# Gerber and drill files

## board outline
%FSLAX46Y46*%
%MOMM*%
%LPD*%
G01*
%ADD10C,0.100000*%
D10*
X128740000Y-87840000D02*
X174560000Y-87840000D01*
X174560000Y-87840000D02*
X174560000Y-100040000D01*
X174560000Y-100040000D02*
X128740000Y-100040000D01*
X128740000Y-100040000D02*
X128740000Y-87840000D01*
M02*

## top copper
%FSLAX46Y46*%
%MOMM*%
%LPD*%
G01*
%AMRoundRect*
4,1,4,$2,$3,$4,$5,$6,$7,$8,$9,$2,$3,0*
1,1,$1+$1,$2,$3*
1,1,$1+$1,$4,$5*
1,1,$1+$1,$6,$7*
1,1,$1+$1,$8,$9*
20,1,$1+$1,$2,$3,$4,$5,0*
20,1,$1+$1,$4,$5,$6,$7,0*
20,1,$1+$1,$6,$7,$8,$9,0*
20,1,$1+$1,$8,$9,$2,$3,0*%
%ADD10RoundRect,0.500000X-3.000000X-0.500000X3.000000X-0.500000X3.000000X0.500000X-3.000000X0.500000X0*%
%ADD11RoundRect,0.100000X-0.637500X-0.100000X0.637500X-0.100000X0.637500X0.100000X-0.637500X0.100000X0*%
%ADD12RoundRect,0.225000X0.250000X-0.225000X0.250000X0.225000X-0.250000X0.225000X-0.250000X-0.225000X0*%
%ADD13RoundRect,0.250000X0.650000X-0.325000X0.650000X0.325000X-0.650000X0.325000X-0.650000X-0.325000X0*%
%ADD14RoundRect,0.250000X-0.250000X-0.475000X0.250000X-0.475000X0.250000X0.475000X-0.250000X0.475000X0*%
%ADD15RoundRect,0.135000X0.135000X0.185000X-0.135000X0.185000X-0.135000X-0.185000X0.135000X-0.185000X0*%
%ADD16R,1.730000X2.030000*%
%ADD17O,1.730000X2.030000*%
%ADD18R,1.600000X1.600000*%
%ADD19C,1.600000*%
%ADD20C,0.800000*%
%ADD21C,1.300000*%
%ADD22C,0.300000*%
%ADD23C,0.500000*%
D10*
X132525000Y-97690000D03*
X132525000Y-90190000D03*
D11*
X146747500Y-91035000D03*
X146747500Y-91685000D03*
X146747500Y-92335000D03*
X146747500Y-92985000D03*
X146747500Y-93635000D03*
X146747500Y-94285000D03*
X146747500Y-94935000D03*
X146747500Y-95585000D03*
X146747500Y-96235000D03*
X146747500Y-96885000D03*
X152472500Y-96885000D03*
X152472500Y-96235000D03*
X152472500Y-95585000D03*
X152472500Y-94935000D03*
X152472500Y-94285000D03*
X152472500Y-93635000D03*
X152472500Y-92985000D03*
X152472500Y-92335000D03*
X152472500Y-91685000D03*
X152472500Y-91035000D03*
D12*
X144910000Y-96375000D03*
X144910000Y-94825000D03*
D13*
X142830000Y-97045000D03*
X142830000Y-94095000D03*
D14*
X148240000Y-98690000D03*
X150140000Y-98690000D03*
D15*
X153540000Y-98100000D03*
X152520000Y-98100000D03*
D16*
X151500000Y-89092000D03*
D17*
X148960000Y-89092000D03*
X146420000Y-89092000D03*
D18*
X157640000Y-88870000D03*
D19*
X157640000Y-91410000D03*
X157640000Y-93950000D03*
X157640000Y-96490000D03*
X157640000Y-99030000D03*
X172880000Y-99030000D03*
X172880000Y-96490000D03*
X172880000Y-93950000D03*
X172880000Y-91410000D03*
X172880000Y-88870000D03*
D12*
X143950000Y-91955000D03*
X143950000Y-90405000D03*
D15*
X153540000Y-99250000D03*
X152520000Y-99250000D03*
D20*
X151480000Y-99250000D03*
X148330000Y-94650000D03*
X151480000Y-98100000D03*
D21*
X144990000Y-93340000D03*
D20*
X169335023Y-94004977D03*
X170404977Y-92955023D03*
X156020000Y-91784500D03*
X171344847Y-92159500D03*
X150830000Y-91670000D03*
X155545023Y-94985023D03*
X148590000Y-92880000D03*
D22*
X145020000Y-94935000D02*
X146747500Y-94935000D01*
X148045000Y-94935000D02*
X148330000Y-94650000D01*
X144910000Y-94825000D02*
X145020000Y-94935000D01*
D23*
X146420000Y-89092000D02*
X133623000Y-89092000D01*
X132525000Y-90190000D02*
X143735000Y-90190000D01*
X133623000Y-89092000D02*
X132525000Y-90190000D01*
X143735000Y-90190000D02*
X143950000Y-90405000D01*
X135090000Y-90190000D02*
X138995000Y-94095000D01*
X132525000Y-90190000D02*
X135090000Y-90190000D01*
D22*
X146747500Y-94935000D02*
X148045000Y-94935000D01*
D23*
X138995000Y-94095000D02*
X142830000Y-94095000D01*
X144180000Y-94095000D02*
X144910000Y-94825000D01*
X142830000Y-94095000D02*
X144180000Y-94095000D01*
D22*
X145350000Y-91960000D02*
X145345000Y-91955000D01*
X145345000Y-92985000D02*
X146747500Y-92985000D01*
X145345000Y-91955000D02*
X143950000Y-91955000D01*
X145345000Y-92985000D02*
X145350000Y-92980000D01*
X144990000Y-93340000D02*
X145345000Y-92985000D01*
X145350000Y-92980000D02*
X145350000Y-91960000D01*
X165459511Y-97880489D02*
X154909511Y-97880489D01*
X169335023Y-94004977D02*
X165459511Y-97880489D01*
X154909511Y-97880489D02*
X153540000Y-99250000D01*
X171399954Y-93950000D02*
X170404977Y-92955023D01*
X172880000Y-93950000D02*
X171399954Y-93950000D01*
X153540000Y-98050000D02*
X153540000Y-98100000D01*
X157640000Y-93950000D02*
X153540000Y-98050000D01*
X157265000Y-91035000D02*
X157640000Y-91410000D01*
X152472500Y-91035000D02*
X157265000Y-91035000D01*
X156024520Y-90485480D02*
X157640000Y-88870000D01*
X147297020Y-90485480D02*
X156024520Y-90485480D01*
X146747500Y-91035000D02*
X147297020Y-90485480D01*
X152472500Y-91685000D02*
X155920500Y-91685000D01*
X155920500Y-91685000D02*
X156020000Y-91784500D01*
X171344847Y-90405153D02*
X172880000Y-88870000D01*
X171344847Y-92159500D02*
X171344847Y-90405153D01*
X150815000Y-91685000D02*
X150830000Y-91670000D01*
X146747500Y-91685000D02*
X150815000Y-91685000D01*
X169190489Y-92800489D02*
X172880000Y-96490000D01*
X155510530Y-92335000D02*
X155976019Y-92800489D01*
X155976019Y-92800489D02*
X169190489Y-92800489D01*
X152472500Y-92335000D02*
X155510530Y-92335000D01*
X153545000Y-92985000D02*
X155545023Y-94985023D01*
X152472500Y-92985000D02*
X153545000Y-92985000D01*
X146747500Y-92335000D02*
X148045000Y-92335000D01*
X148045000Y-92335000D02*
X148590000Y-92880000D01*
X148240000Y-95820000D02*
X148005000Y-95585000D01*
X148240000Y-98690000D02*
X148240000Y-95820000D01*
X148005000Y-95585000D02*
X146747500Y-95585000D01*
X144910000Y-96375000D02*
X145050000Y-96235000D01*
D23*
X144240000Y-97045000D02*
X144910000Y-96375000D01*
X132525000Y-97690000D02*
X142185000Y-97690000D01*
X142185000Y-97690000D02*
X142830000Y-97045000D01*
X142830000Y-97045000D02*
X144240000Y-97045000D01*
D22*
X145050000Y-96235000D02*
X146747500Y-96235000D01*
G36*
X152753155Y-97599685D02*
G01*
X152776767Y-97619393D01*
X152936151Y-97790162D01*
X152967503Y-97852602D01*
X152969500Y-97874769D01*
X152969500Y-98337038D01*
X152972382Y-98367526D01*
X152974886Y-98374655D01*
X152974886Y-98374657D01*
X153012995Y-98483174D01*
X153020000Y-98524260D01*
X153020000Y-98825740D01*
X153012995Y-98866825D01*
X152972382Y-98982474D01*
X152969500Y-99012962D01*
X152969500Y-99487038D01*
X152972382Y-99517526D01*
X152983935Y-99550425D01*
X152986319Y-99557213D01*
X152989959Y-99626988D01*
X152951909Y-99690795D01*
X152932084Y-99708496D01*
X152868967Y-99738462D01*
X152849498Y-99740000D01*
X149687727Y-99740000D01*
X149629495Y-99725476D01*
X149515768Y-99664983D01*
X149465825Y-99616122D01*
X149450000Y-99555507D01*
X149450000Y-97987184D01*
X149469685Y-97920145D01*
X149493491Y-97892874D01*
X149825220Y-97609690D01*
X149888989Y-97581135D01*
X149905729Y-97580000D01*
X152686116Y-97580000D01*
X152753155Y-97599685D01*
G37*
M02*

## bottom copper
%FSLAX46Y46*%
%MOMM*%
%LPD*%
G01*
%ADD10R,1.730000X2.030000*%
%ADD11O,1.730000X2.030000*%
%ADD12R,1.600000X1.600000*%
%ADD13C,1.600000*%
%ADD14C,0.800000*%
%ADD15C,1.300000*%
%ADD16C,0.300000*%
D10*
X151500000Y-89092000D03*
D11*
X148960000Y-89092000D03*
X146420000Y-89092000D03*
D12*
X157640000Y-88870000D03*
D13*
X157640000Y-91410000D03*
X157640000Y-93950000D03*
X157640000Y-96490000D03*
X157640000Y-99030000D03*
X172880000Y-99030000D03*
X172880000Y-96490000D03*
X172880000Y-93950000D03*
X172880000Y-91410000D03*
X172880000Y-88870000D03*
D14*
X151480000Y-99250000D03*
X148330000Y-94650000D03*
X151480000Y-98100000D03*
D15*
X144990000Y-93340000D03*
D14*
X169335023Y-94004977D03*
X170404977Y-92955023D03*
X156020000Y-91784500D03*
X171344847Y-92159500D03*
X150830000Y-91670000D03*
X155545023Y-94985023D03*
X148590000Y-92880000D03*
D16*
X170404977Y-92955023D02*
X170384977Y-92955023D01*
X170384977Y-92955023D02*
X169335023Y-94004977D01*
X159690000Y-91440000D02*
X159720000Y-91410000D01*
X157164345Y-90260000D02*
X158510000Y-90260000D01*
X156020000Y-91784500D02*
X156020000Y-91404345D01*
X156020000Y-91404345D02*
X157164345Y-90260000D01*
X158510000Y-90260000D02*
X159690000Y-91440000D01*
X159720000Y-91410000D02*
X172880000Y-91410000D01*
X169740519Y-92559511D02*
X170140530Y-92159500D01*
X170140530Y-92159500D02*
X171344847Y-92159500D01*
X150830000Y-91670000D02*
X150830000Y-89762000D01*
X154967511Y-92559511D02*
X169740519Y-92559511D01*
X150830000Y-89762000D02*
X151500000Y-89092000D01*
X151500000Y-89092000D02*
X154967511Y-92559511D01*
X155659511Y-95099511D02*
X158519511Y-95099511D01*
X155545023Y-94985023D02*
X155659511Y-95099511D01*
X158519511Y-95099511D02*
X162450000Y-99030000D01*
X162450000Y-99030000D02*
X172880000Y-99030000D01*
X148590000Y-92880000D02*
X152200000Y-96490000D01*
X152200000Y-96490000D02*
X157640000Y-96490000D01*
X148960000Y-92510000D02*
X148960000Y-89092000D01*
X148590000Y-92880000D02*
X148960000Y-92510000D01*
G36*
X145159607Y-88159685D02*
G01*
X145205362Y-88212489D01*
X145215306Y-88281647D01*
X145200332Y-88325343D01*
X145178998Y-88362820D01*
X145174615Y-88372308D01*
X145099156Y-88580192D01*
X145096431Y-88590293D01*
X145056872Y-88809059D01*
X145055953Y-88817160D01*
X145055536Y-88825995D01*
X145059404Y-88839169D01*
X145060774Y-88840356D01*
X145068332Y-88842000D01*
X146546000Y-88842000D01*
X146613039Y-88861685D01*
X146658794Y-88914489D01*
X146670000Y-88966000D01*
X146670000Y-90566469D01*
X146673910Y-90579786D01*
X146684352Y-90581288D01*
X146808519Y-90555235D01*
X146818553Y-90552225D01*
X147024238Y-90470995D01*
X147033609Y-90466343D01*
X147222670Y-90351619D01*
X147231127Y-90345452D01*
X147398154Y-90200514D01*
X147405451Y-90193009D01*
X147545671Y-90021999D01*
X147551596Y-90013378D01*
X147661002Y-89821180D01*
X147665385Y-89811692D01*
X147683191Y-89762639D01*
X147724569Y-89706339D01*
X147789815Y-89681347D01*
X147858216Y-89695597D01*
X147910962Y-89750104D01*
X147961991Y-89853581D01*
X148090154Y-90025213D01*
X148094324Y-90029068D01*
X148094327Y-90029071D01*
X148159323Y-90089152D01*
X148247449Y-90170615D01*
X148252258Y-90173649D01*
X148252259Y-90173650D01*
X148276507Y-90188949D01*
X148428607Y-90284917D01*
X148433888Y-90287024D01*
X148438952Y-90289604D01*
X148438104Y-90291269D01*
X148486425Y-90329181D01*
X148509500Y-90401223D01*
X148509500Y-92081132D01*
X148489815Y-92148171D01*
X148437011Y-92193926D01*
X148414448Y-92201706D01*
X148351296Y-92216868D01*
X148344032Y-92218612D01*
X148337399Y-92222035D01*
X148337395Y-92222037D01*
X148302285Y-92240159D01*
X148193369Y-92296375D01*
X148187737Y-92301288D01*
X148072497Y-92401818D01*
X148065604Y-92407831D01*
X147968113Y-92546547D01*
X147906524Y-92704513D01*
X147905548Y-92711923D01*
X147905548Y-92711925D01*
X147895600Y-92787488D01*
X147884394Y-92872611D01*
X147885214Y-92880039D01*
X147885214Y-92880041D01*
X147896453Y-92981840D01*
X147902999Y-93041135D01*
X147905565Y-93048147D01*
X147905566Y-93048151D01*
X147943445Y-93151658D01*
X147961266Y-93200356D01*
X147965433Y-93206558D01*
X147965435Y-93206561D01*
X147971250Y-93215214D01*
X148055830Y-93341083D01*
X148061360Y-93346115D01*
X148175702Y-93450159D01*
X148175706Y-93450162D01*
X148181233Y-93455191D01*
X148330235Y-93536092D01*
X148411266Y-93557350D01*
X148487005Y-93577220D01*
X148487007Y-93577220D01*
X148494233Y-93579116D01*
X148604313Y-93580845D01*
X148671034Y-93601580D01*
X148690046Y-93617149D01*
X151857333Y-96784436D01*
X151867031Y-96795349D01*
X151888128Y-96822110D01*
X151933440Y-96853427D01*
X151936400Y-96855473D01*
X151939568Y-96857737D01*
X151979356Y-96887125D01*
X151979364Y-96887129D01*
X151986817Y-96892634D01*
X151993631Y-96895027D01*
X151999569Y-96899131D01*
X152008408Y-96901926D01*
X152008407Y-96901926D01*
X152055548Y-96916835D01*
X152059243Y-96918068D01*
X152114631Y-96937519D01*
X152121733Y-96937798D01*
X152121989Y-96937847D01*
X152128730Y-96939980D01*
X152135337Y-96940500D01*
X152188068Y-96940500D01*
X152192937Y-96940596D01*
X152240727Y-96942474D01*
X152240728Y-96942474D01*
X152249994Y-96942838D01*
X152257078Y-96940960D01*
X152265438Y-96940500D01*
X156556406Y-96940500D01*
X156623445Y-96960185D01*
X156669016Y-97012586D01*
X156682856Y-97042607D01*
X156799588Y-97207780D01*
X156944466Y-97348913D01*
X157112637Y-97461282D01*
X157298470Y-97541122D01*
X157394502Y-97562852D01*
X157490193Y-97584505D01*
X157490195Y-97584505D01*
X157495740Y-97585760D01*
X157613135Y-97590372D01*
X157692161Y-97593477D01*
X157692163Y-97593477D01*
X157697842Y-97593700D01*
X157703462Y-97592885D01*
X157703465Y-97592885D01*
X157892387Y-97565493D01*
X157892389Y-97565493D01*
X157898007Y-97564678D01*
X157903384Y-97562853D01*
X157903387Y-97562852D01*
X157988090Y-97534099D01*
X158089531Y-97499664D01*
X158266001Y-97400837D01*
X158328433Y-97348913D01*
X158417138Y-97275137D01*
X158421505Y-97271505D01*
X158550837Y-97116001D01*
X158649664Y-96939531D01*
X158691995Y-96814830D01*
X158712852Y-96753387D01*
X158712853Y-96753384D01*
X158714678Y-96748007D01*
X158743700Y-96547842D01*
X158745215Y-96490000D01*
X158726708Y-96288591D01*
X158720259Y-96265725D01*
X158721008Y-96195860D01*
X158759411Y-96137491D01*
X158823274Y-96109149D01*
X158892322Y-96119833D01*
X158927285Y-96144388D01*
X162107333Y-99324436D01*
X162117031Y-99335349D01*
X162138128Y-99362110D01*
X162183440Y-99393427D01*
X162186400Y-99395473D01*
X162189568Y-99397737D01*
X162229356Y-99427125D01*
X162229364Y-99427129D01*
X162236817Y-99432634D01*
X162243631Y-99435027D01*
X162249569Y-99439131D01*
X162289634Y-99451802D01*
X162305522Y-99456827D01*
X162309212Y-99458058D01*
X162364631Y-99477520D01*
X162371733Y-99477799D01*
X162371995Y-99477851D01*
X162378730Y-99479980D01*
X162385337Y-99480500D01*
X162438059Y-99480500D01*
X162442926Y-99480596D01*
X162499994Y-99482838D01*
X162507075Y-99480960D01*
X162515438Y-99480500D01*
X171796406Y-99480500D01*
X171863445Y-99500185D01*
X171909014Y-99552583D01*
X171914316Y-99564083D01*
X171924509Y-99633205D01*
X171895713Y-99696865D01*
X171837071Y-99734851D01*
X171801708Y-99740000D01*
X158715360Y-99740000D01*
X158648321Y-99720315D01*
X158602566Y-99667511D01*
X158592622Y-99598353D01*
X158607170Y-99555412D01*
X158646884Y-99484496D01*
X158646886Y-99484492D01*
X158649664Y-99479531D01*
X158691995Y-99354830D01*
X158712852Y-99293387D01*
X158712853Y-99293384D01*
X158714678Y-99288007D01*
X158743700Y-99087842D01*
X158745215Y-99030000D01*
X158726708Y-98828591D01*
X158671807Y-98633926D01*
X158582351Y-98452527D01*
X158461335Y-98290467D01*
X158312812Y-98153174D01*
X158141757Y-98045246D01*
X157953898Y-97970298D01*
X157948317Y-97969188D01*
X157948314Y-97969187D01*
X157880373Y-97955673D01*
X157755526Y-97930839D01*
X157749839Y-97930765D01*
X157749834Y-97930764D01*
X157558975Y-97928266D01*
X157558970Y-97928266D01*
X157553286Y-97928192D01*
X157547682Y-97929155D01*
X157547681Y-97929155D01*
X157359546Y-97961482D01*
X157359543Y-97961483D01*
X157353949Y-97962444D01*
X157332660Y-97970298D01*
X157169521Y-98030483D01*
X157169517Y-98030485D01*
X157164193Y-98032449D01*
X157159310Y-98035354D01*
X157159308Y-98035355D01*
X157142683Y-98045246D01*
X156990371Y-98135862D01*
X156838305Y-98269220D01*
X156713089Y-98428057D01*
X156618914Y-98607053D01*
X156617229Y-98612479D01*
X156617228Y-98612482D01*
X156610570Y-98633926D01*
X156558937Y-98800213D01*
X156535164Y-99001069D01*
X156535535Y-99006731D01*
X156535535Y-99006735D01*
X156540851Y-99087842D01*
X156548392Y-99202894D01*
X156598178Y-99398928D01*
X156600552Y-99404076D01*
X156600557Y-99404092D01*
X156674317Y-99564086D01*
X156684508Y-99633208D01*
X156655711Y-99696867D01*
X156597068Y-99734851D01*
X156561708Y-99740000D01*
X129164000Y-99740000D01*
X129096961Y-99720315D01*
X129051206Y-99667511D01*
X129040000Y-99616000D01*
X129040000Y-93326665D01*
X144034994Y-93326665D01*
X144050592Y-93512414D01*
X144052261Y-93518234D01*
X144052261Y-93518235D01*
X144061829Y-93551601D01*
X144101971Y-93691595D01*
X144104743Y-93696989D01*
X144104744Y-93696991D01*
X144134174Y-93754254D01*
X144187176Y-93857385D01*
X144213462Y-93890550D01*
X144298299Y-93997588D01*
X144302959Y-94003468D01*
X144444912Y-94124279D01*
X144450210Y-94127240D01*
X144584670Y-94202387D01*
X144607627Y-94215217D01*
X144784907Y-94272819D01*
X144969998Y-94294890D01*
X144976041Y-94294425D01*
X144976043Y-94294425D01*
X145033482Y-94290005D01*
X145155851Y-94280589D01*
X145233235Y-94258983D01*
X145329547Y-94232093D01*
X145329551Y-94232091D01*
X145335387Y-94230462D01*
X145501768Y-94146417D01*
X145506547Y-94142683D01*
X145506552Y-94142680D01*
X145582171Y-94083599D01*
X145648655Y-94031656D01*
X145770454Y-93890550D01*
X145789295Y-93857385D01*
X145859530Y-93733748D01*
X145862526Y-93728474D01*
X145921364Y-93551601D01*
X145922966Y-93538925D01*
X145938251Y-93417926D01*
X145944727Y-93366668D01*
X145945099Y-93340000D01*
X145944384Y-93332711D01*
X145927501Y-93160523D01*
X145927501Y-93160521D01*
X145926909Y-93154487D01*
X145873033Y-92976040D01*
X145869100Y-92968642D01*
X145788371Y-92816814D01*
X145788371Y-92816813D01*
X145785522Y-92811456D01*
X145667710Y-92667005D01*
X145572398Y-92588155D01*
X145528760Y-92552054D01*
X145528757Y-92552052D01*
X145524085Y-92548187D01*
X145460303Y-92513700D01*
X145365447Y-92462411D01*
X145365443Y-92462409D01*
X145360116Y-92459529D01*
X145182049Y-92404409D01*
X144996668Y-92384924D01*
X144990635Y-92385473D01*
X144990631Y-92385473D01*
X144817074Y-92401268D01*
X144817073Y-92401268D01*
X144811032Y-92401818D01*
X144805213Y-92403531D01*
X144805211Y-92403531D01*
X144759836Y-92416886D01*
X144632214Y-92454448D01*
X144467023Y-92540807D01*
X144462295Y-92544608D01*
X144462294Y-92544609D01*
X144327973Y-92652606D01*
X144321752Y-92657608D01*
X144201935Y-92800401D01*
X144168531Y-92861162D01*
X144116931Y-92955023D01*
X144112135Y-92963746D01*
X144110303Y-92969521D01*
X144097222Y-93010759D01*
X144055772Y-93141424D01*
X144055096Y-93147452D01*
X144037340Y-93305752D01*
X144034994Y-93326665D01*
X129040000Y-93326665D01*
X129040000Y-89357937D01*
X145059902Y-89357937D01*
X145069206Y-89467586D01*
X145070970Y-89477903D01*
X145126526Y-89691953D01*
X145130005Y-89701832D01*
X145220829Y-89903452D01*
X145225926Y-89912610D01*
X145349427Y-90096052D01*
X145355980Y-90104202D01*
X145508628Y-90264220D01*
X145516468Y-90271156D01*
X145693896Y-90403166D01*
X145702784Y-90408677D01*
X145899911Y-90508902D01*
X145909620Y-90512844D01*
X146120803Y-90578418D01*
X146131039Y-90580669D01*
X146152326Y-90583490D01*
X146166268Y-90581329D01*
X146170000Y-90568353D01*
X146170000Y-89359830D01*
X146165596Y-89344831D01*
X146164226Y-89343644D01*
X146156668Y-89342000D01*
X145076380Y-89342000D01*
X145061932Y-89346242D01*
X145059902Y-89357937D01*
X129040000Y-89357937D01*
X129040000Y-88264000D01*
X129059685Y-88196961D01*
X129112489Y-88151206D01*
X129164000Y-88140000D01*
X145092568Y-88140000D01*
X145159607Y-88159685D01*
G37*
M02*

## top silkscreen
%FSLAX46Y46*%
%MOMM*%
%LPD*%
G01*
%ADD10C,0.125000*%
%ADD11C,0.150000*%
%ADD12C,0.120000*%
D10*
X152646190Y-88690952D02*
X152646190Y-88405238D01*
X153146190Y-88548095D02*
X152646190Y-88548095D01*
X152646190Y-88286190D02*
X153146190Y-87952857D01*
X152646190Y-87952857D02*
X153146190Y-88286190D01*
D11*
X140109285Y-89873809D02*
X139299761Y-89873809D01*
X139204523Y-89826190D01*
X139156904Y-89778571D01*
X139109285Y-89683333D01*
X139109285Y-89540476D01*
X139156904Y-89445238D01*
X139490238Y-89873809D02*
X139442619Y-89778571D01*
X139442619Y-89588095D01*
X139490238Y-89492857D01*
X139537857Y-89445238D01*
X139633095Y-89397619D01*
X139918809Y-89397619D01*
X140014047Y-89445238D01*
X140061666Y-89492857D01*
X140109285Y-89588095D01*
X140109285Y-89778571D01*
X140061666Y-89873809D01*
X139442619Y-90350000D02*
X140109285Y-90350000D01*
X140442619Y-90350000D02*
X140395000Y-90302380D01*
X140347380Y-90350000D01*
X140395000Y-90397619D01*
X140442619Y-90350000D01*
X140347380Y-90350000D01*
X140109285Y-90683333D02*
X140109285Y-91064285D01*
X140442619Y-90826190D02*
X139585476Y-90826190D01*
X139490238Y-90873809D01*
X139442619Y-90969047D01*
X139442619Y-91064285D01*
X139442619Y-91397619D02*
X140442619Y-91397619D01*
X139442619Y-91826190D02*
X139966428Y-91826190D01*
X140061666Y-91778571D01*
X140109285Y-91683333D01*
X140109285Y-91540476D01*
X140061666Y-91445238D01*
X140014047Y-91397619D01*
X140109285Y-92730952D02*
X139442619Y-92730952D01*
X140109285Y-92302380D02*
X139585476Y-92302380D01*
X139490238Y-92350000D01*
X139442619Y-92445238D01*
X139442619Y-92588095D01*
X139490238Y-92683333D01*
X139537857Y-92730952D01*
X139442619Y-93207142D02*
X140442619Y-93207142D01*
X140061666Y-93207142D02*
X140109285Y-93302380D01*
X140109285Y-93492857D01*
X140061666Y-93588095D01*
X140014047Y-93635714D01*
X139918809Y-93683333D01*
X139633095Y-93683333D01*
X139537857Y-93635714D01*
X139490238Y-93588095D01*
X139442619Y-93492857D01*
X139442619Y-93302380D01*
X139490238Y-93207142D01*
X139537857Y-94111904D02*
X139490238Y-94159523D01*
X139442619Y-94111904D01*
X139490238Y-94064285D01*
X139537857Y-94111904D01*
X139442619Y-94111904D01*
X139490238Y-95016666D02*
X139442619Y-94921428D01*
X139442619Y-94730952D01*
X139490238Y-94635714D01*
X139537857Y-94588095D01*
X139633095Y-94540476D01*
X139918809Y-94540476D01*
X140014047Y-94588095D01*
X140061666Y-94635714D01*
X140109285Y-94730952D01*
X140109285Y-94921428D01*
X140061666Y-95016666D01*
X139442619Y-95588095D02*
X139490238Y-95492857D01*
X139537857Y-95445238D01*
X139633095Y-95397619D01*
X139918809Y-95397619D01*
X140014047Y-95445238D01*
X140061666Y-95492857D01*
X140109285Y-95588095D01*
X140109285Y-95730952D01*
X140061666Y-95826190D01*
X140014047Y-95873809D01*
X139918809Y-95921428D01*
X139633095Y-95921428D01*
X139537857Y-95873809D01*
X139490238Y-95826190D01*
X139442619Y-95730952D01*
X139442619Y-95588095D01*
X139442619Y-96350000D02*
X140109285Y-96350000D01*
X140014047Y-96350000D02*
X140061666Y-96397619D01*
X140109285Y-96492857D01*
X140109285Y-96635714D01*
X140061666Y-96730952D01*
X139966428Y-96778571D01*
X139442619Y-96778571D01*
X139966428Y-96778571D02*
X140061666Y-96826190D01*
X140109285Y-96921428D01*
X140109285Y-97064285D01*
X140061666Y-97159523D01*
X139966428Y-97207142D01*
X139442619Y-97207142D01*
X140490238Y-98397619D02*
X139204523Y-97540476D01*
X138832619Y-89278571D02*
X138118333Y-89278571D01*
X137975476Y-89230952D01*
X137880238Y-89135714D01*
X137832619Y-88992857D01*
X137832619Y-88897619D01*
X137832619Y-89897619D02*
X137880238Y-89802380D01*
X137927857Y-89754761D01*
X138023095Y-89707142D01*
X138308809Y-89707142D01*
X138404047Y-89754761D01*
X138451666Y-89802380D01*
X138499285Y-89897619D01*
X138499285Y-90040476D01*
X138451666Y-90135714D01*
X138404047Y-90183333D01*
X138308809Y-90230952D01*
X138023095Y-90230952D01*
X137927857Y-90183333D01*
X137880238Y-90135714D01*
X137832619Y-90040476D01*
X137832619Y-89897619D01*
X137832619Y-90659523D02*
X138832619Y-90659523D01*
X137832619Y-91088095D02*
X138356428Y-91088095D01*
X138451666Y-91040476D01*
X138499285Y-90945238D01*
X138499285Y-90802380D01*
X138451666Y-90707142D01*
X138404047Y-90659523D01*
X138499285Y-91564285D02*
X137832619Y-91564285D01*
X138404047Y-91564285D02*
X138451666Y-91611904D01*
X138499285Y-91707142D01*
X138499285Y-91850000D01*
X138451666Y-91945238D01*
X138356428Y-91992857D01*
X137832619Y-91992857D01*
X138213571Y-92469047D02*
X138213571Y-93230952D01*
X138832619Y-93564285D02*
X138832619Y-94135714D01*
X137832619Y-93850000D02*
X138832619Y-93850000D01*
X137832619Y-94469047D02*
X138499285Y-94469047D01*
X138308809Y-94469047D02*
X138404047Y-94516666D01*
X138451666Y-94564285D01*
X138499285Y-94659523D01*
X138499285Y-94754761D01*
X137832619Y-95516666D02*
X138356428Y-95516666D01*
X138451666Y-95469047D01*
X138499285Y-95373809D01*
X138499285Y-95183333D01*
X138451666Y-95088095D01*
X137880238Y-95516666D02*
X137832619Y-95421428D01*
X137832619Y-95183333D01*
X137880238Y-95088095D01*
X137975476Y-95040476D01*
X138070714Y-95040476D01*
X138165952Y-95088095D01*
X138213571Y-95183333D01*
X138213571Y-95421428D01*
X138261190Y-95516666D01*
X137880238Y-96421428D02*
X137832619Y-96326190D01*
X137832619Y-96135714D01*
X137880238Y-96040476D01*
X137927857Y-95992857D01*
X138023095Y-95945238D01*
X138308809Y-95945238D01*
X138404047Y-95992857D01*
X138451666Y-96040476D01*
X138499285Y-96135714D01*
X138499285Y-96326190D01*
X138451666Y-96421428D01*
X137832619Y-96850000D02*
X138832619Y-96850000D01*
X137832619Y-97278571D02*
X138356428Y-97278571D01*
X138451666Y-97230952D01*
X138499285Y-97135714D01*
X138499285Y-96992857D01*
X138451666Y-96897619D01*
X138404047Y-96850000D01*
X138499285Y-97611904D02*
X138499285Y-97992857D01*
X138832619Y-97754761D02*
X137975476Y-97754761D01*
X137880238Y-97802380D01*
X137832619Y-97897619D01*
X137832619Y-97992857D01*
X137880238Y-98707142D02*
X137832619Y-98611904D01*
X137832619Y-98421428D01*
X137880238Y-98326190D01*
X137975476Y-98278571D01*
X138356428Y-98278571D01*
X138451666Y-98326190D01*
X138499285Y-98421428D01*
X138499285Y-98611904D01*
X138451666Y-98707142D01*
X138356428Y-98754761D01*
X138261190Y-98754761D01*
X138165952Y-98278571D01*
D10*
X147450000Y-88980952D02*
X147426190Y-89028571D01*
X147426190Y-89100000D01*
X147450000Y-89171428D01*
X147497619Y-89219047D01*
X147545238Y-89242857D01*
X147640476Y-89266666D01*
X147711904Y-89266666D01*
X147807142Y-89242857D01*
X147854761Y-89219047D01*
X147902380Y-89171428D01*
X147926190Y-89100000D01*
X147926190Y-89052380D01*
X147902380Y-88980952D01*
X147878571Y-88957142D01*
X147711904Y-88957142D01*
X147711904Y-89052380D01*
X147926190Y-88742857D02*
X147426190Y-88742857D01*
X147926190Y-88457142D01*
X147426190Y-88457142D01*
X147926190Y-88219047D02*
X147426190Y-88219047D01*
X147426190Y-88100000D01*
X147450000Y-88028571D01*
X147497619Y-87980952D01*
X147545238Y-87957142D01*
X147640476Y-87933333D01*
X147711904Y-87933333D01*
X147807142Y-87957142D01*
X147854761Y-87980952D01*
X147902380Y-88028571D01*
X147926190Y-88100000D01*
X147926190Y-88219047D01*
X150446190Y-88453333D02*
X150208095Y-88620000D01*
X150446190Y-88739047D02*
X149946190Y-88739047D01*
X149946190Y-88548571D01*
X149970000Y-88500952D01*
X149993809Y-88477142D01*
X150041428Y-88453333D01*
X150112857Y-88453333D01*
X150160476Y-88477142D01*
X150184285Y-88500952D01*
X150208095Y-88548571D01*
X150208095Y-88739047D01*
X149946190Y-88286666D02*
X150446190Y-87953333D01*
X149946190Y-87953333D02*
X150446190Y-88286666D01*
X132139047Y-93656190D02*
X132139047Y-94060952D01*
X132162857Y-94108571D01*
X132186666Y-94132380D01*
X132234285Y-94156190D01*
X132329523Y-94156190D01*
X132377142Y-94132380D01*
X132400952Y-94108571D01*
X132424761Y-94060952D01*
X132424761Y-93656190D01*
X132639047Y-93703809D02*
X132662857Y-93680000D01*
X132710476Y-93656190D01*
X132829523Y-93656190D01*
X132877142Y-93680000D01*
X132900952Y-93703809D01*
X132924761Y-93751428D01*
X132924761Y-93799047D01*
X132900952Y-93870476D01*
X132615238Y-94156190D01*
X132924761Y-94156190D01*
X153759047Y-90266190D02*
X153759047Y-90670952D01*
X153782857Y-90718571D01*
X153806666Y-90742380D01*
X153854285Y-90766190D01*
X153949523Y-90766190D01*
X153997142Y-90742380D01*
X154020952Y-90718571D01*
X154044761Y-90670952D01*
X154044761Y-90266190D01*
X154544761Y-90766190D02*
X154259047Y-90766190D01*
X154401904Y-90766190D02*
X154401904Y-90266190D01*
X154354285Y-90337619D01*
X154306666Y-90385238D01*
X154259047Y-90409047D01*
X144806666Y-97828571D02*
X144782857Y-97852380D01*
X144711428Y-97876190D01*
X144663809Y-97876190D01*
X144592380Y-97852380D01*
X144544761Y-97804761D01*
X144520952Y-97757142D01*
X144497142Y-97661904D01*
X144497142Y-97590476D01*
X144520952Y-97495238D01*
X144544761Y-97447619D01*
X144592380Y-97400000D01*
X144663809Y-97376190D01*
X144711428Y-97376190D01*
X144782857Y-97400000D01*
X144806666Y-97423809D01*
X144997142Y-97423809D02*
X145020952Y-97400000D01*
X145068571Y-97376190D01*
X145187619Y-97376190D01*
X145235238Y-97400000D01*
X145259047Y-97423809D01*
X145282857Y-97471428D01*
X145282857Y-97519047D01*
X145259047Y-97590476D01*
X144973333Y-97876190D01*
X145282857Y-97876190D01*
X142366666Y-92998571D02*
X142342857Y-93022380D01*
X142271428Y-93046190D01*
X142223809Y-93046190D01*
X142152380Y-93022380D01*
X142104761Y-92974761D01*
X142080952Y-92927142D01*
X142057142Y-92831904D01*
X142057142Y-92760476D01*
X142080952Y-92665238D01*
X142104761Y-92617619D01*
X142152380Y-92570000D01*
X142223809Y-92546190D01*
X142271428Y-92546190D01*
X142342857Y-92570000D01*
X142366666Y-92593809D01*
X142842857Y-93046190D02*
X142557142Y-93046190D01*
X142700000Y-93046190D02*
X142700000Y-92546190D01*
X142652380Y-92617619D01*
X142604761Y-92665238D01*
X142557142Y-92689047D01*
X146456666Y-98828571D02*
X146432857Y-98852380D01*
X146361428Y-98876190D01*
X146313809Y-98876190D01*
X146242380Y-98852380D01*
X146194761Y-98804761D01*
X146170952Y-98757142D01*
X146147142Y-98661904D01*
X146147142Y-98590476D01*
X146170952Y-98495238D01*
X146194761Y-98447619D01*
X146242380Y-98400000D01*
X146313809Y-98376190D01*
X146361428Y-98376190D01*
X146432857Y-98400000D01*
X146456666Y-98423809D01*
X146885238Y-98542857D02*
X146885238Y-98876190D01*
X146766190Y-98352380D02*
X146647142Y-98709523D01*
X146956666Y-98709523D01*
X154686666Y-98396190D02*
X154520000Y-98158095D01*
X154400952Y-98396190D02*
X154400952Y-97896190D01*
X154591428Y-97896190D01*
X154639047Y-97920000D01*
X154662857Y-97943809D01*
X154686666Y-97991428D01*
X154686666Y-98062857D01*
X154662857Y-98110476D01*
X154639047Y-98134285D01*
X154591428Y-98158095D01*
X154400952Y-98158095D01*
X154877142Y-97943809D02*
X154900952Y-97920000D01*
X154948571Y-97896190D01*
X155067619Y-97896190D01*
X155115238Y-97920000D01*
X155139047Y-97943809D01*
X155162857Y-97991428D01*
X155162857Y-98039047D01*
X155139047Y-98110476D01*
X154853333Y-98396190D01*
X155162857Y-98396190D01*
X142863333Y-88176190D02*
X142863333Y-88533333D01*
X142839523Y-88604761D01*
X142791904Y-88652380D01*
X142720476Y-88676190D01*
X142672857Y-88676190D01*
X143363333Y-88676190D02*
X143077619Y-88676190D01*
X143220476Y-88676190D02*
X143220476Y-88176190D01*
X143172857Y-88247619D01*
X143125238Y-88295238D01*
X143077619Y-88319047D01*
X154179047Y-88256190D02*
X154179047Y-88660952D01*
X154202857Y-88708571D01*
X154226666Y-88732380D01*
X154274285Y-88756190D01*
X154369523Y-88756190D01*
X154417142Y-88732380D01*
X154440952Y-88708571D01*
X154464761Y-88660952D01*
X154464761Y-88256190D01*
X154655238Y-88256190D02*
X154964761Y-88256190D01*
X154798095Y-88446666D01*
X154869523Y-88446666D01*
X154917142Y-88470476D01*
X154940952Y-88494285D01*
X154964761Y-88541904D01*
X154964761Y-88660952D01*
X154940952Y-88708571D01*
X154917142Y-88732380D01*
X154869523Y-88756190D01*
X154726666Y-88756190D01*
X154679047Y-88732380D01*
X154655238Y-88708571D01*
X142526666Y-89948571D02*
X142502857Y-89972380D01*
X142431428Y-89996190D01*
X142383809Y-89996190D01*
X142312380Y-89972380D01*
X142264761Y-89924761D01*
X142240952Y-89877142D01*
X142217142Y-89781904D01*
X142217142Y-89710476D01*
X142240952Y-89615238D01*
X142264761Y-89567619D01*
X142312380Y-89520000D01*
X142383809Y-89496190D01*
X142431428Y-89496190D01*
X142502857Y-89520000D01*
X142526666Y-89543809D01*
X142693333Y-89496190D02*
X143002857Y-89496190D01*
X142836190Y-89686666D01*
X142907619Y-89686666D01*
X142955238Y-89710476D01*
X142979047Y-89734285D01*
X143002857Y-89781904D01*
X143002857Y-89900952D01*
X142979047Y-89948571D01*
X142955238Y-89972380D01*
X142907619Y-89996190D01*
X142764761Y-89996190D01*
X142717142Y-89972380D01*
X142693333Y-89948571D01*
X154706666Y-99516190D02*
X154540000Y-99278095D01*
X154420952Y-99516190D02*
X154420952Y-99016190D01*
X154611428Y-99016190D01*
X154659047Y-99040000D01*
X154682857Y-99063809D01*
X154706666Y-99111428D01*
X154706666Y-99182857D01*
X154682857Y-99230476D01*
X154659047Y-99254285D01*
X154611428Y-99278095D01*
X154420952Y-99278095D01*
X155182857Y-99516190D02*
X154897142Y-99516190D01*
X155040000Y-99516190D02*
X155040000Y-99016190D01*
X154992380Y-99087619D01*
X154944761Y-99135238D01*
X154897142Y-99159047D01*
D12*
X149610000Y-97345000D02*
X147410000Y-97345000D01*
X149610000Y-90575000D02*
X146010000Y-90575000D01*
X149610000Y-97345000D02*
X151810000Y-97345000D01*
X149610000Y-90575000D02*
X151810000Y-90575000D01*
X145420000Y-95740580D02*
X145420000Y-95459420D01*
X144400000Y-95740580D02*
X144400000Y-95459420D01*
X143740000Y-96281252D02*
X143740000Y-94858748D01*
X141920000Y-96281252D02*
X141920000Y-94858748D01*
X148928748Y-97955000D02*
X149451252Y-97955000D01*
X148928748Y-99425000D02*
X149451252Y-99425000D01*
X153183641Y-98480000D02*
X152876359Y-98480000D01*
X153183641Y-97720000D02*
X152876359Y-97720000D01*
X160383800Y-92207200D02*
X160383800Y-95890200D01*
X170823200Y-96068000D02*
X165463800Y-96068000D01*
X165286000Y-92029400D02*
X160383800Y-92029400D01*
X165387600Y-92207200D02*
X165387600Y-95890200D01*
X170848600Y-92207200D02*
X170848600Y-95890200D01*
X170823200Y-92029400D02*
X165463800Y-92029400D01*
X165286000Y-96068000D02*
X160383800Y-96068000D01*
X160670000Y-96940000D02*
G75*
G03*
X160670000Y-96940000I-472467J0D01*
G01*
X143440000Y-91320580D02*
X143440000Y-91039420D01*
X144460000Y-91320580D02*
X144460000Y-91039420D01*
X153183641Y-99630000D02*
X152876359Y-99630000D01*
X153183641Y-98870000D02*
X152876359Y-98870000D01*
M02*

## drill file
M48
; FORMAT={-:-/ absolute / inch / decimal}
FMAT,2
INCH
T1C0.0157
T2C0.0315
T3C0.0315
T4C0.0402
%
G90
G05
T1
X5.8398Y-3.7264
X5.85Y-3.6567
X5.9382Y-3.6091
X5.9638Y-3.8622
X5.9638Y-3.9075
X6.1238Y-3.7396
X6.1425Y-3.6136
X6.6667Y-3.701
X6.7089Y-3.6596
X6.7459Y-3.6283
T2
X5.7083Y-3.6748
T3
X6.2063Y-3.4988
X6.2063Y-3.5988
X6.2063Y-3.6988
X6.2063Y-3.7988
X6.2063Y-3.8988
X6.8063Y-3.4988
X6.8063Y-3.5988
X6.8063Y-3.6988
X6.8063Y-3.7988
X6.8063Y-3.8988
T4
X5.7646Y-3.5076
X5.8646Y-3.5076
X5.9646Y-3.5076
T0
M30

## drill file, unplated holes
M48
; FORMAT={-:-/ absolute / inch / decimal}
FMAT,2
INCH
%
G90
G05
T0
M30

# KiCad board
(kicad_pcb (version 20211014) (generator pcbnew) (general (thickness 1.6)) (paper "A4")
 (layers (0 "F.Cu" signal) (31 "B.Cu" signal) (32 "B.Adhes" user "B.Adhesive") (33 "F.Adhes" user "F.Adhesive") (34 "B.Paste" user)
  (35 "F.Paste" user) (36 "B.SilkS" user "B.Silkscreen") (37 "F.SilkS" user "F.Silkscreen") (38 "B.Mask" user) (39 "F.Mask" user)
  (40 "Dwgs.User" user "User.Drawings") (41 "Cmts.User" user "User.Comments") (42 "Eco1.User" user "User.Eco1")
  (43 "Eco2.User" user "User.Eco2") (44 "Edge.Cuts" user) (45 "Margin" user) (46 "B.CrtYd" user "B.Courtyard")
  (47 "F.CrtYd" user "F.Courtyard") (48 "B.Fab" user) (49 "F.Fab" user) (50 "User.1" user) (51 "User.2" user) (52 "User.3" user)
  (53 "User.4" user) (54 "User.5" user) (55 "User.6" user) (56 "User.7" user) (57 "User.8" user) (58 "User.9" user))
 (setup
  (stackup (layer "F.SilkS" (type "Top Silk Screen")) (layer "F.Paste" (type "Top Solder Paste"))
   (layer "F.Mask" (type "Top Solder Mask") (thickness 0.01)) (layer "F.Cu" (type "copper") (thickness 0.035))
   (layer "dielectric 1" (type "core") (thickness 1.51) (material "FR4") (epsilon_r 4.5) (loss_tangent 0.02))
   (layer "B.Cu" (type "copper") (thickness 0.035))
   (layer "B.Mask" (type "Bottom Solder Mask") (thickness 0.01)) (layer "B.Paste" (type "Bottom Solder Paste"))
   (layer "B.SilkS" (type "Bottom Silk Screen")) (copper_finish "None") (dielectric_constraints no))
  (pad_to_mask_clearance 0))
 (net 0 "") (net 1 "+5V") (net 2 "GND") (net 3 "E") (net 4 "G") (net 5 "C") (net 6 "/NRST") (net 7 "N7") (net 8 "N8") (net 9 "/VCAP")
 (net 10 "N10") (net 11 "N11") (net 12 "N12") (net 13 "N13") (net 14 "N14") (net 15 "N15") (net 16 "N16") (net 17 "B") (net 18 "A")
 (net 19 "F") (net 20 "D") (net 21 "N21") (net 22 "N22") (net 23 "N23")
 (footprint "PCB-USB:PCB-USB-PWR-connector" (layer "F.Cu") (at 132.525 93.94)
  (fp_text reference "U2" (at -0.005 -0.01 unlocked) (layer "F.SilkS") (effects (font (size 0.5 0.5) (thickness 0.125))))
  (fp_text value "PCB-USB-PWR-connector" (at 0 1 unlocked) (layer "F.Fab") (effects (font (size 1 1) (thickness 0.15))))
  (pad "1" smd roundrect (at 0 3.75) (size 7 2) (layers "F.Cu" "F.Paste" "F.Mask") (roundrect_rratio 0.25) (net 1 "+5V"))
  (pad "2" smd roundrect (at 0 -3.75) (size 7 2) (layers "F.Cu" "F.Paste" "F.Mask") (roundrect_rratio 0.25) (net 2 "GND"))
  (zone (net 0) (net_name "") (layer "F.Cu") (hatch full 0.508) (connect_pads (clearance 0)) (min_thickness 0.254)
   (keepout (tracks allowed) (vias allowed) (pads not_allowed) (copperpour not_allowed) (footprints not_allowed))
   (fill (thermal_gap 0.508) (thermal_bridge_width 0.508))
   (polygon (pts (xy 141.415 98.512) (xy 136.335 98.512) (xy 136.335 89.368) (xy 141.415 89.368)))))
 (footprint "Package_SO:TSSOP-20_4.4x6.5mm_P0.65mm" (layer "F.Cu") (at 149.61 93.96)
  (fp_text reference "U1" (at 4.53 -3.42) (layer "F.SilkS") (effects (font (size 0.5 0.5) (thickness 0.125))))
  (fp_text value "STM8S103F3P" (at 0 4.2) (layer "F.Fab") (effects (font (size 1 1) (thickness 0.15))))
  (fp_line (start 0 3.385) (end -2.2 3.385) (layer "F.SilkS") (width 0.12))
  (fp_line (start 0 -3.385) (end -3.6 -3.385) (layer "F.SilkS") (width 0.12))
  (fp_line (start 0 3.385) (end 2.2 3.385) (layer "F.SilkS") (width 0.12))
  (fp_line (start 0 -3.385) (end 2.2 -3.385) (layer "F.SilkS") (width 0.12))
  (pad "1" smd roundrect (at -2.8625 -2.925) (size 1.475 0.4) (layers "F.Cu" "F.Paste" "F.Mask") (roundrect_rratio 0.25) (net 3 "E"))
  (pad "2" smd roundrect (at -2.8625 -2.275) (size 1.475 0.4) (layers "F.Cu" "F.Paste" "F.Mask") (roundrect_rratio 0.25) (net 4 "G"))
  (pad "3" smd roundrect (at -2.8625 -1.625) (size 1.475 0.4) (layers "F.Cu" "F.Paste" "F.Mask") (roundrect_rratio 0.25) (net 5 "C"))
  (pad "4" smd roundrect (at -2.8625 -0.975) (size 1.475 0.4) (layers "F.Cu" "F.Paste" "F.Mask") (roundrect_rratio 0.25) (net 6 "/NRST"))
  (pad "5" smd roundrect (at -2.8625 -0.325) (size 1.475 0.4) (layers "F.Cu" "F.Paste" "F.Mask") (roundrect_rratio 0.25) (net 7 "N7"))
  (pad "6" smd roundrect (at -2.8625 0.325) (size 1.475 0.4) (layers "F.Cu" "F.Paste" "F.Mask") (roundrect_rratio 0.25) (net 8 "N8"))
  (pad "7" smd roundrect (at -2.8625 0.975) (size 1.475 0.4) (layers "F.Cu" "F.Paste" "F.Mask") (roundrect_rratio 0.25) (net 2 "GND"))
  (pad "8" smd roundrect (at -2.8625 1.625) (size 1.475 0.4) (layers "F.Cu" "F.Paste" "F.Mask") (roundrect_rratio 0.25) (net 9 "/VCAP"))
  (pad "9" smd roundrect (at -2.8625 2.275) (size 1.475 0.4) (layers "F.Cu" "F.Paste" "F.Mask") (roundrect_rratio 0.25) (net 1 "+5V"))
  (pad "10" smd roundrect (at -2.8625 2.925) (size 1.475 0.4) (layers "F.Cu" "F.Paste" "F.Mask") (roundrect_rratio 0.25) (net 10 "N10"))
  (pad "11" smd roundrect (at 2.8625 2.925) (size 1.475 0.4) (layers "F.Cu" "F.Paste" "F.Mask") (roundrect_rratio 0.25) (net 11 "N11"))
  (pad "12" smd roundrect (at 2.8625 2.275) (size 1.475 0.4) (layers "F.Cu" "F.Paste" "F.Mask") (roundrect_rratio 0.25) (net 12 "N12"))
  (pad "13" smd roundrect (at 2.8625 1.625) (size 1.475 0.4) (layers "F.Cu" "F.Paste" "F.Mask") (roundrect_rratio 0.25) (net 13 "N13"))
  (pad "14" smd roundrect (at 2.8625 0.975) (size 1.475 0.4) (layers "F.Cu" "F.Paste" "F.Mask") (roundrect_rratio 0.25) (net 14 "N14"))
  (pad "15" smd roundrect (at 2.8625 0.325) (size 1.475 0.4) (layers "F.Cu" "F.Paste" "F.Mask") (roundrect_rratio 0.25) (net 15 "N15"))
  (pad "16" smd roundrect (at 2.8625 -0.325) (size 1.475 0.4) (layers "F.Cu" "F.Paste" "F.Mask") (roundrect_rratio 0.25) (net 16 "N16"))
  (pad "17" smd roundrect (at 2.8625 -0.975) (size 1.475 0.4) (layers "F.Cu" "F.Paste" "F.Mask") (roundrect_rratio 0.25) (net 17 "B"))
  (pad "18" smd roundrect (at 2.8625 -1.625) (size 1.475 0.4) (layers "F.Cu" "F.Paste" "F.Mask") (roundrect_rratio 0.25) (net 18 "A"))
  (pad "19" smd roundrect (at 2.8625 -2.275) (size 1.475 0.4) (layers "F.Cu" "F.Paste" "F.Mask") (roundrect_rratio 0.25) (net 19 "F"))
  (pad "20" smd roundrect (at 2.8625 -2.925) (size 1.475 0.4) (layers "F.Cu" "F.Paste" "F.Mask") (roundrect_rratio 0.25) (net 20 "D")))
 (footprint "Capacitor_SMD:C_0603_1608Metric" (layer "F.Cu") (at 144.91 95.6 90)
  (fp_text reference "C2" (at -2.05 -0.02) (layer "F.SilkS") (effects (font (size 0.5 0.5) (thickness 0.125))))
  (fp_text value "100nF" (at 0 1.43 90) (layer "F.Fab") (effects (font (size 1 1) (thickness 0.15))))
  (fp_line (start -0.14058 0.51) (end 0.14058 0.51) (layer "F.SilkS") (width 0.12))
  (fp_line (start -0.14058 -0.51) (end 0.14058 -0.51) (layer "F.SilkS") (width 0.12))
  (pad "1" smd roundrect (at -0.775 0 90) (size 0.9 0.95) (layers "F.Cu" "F.Paste" "F.Mask") (roundrect_rratio 0.25) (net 1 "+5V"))
  (pad "2" smd roundrect (at 0.775 0 90) (size 0.9 0.95) (layers "F.Cu" "F.Paste" "F.Mask") (roundrect_rratio 0.25) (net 2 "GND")))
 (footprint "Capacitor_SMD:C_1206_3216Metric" (layer "F.Cu") (at 142.83 95.57 90)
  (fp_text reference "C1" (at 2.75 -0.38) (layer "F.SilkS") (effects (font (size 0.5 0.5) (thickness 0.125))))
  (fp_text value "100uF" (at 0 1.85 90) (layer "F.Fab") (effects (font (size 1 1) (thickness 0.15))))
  (fp_line (start -0.711252 0.91) (end 0.711252 0.91) (layer "F.SilkS") (width 0.12))
  (fp_line (start -0.711252 -0.91) (end 0.711252 -0.91) (layer "F.SilkS") (width 0.12))
  (pad "1" smd roundrect (at -1.475 0 90) (size 1.15 1.8) (layers "F.Cu" "F.Paste" "F.Mask") (roundrect_rratio 0.2173913043) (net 1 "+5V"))
  (pad "2" smd roundrect (at 1.475 0 90) (size 1.15 1.8) (layers "F.Cu" "F.Paste" "F.Mask") (roundrect_rratio 0.2173913043) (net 2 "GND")))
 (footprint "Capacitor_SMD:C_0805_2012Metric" (layer "F.Cu") (at 149.19 98.69)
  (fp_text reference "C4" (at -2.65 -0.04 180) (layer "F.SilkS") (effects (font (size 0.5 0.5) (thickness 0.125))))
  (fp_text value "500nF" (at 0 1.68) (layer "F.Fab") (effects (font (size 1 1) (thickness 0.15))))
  (fp_line (start -0.261252 -0.735) (end 0.261252 -0.735) (layer "F.SilkS") (width 0.12))
  (fp_line (start -0.261252 0.735) (end 0.261252 0.735) (layer "F.SilkS") (width 0.12))
  (pad "1" smd roundrect (at -0.95 0) (size 1 1.45) (layers "F.Cu" "F.Paste" "F.Mask") (roundrect_rratio 0.25) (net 9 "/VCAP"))
  (pad "2" smd roundrect (at 0.95 0) (size 1 1.45) (layers "F.Cu" "F.Paste" "F.Mask") (roundrect_rratio 0.25) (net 2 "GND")))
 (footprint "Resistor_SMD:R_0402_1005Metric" (layer "F.Cu") (at 153.03 98.1 180)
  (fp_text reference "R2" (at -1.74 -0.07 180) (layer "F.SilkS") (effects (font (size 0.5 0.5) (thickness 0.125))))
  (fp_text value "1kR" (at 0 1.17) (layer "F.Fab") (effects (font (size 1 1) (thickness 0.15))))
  (fp_line (start -0.153641 -0.38) (end 0.153641 -0.38) (layer "F.SilkS") (width 0.12))
  (fp_line (start -0.153641 0.38) (end 0.153641 0.38) (layer "F.SilkS") (width 0.12))
  (pad "1" smd roundrect (at -0.51 0 180) (size 0.54 0.64) (layers "F.Cu" "F.Paste" "F.Mask") (roundrect_rratio 0.25) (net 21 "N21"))
  (pad "2" smd roundrect (at 0.51 0 180) (size 0.54 0.64) (layers "F.Cu" "F.Paste" "F.Mask") (roundrect_rratio 0.25) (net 2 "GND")))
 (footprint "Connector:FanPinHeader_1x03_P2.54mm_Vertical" (layer "F.Cu") (at 151.5 89.092 180)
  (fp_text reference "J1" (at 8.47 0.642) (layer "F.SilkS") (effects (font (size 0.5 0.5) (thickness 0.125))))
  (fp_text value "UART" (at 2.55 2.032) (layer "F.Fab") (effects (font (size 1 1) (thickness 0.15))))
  (pad "1" thru_hole rect (at 0 0 270) (size 2.03 1.73) (drill 1.02) (layers *.Cu *.Mask) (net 4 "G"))
  (pad "2" thru_hole oval (at 2.54 0 270) (size 2.03 1.73) (drill 1.02) (layers *.Cu *.Mask) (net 5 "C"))
  (pad "3" thru_hole oval (at 5.08 0 270) (size 2.03 1.73) (drill 1.02) (layers *.Cu *.Mask) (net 2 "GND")))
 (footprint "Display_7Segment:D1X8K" (layer "F.Cu") (at 157.64 88.87)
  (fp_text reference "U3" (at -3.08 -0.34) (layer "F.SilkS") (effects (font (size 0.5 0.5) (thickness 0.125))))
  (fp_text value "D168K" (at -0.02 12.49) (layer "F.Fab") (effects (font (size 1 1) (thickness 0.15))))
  (fp_line (start 2.7438 3.3372) (end 2.7438 7.0202) (layer "F.SilkS") (width 0.12))
  (fp_line (start 13.1832 7.198) (end 7.8238 7.198) (layer "F.SilkS") (width 0.12))
  (fp_line (start 7.646 3.1594) (end 2.7438 3.1594) (layer "F.SilkS") (width 0.12))
  (fp_line (start 7.7476 3.3372) (end 7.7476 7.0202) (layer "F.SilkS") (width 0.12))
  (fp_line (start 13.2086 3.3372) (end 13.2086 7.0202) (layer "F.SilkS") (width 0.12))
  (fp_line (start 13.1832 3.1594) (end 7.8238 3.1594) (layer "F.SilkS") (width 0.12))
  (fp_line (start 7.646 7.198) (end 2.7438 7.198) (layer "F.SilkS") (width 0.12))
  (fp_circle (center 2.557533 8.07) (end 2.836933 7.689) (layer "F.SilkS") (width 0.12) (fill none))
  (pad "1" thru_hole rect (at 0 0 270) (size 1.6 1.6) (drill 0.8) (layers *.Cu *.Mask) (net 3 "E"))
  (pad "2" thru_hole circle (at 0 2.54 270) (size 1.6 1.6) (drill 0.8) (layers *.Cu *.Mask) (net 20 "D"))
  (pad "3" thru_hole circle (at 0 5.08 270) (size 1.6 1.6) (drill 0.8) (layers *.Cu *.Mask) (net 21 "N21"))
  (pad "4" thru_hole circle (at 0 7.62 270) (size 1.6 1.6) (drill 0.8) (layers *.Cu *.Mask) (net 5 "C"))
  (pad "5" thru_hole circle (at 0 10.16 270) (size 1.6 1.6) (drill 0.8) (layers *.Cu *.Mask) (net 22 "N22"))
  (pad "6" thru_hole circle (at 15.24 10.16 270) (size 1.6 1.6) (drill 0.8) (layers *.Cu *.Mask) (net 17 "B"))
  (pad "7" thru_hole circle (at 15.24 7.62 270) (size 1.6 1.6) (drill 0.8) (layers *.Cu *.Mask) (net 18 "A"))
  (pad "8" thru_hole circle (at 15.24 5.08 270) (size 1.6 1.6) (drill 0.8) (layers *.Cu *.Mask) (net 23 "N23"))
  (pad "9" thru_hole circle (at 15.24 2.54 270) (size 1.6 1.6) (drill 0.8) (layers *.Cu *.Mask) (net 19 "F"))
  (pad "10" thru_hole circle (at 15.24 0 270) (size 1.6 1.6) (drill 0.8) (layers *.Cu *.Mask) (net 4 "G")))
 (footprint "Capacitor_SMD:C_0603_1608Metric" (layer "F.Cu") (at 143.95 91.18 90)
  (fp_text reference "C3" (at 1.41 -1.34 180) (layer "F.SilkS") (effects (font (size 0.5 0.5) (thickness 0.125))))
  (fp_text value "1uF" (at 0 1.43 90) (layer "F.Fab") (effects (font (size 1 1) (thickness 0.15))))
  (fp_line (start -0.14058 -0.51) (end 0.14058 -0.51) (layer "F.SilkS") (width 0.12))
  (fp_line (start -0.14058 0.51) (end 0.14058 0.51) (layer "F.SilkS") (width 0.12))
  (pad "1" smd roundrect (at -0.775 0 90) (size 0.9 0.95) (layers "F.Cu" "F.Paste" "F.Mask") (roundrect_rratio 0.25) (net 6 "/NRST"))
  (pad "2" smd roundrect (at 0.775 0 90) (size 0.9 0.95) (layers "F.Cu" "F.Paste" "F.Mask") (roundrect_rratio 0.25) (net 2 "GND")))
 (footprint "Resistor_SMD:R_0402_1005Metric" (layer "F.Cu") (at 153.03 99.25 180)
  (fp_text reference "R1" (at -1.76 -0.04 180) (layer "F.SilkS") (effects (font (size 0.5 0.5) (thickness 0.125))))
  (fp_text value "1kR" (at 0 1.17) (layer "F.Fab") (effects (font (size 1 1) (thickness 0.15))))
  (fp_line (start -0.153641 -0.38) (end 0.153641 -0.38) (layer "F.SilkS") (width 0.12))
  (fp_line (start -0.153641 0.38) (end 0.153641 0.38) (layer "F.SilkS") (width 0.12))
  (pad "1" smd roundrect (at -0.51 0 180) (size 0.54 0.64) (layers "F.Cu" "F.Paste" "F.Mask") (roundrect_rratio 0.25) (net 23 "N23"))
  (pad "2" smd roundrect (at 0.51 0 180) (size 0.54 0.64) (layers "F.Cu" "F.Paste" "F.Mask") (roundrect_rratio 0.25) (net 2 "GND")))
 (gr_rect (start 128.74 87.84) (end 174.56 100.04) (layer "Edge.Cuts") (width 0.1) (fill none))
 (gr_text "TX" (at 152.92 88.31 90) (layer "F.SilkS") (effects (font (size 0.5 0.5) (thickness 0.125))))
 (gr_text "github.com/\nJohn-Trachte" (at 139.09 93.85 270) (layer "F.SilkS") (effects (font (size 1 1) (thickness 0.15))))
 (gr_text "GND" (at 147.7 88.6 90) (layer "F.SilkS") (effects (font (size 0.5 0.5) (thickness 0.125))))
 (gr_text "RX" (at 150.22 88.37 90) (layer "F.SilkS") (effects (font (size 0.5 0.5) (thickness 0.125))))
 (segment (start 145.02 94.935) (end 146.7475 94.935) (width 0.3) (layer "F.Cu") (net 2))
 (segment (start 148.045 94.935) (end 148.33 94.65) (width 0.3) (layer "F.Cu") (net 2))
 (segment (start 144.91 94.825) (end 145.02 94.935) (width 0.3) (layer "F.Cu") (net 2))
 (segment (start 146.42 89.092) (end 133.623 89.092) (width 0.5) (layer "F.Cu") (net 2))
 (segment (start 132.525 90.19) (end 143.735 90.19) (width 0.5) (layer "F.Cu") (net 2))
 (segment (start 133.623 89.092) (end 132.525 90.19) (width 0.5) (layer "F.Cu") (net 2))
 (segment (start 143.735 90.19) (end 143.95 90.405) (width 0.5) (layer "F.Cu") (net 2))
 (segment (start 135.09 90.19) (end 138.995 94.095) (width 0.5) (layer "F.Cu") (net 2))
 (segment (start 132.525 90.19) (end 135.09 90.19) (width 0.5) (layer "F.Cu") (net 2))
 (segment (start 146.7475 94.935) (end 148.045 94.935) (width 0.3) (layer "F.Cu") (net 2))
 (segment (start 138.995 94.095) (end 142.83 94.095) (width 0.5) (layer "F.Cu") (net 2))
 (segment (start 144.18 94.095) (end 144.91 94.825) (width 0.5) (layer "F.Cu") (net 2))
 (segment (start 142.83 94.095) (end 144.18 94.095) (width 0.5) (layer "F.Cu") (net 2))
 (via (at 151.48 99.25) (size 0.8) (drill 0.4) (layers "F.Cu" "B.Cu") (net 2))
 (via (at 148.33 94.65) (size 0.8) (drill 0.4) (layers "F.Cu" "B.Cu") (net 2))
 (via (at 151.48 98.1) (size 0.8) (drill 0.4) (layers "F.Cu" "B.Cu") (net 2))
 (segment (start 145.35 91.96) (end 145.345 91.955) (width 0.3) (layer "F.Cu") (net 6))
 (segment (start 145.345 92.985) (end 146.7475 92.985) (width 0.3) (layer "F.Cu") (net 6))
 (segment (start 145.345 91.955) (end 143.95 91.955) (width 0.3) (layer "F.Cu") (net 6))
 (segment (start 145.345 92.985) (end 145.35 92.98) (width 0.3) (layer "F.Cu") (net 6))
 (segment (start 144.99 93.34) (end 145.345 92.985) (width 0.3) (layer "F.Cu") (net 6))
 (segment (start 145.35 92.98) (end 145.35 91.96) (width 0.3) (layer "F.Cu") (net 6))
 (via (at 144.99 93.34) (size 1.3) (drill 0.8) (layers "F.Cu" "B.Cu") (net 6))
 (segment (start 165.459511 97.880489) (end 154.909511 97.880489) (width 0.3) (layer "F.Cu") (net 23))
 (segment (start 169.335023 94.004977) (end 165.459511 97.880489) (width 0.3) (layer "F.Cu") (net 23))
 (segment (start 154.909511 97.880489) (end 153.54 99.25) (width 0.3) (layer "F.Cu") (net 23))
 (segment (start 171.399954 93.95) (end 170.404977 92.955023) (width 0.3) (layer "F.Cu") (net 23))
 (segment (start 172.88 93.95) (end 171.399954 93.95) (width 0.3) (layer "F.Cu") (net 23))
 (via (at 169.335023 94.004977) (size 0.8) (drill 0.4) (layers "F.Cu" "B.Cu") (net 23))
 (via (at 170.404977 92.955023) (size 0.8) (drill 0.4) (layers "F.Cu" "B.Cu") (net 23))
 (segment (start 170.404977 92.955023) (end 170.384977 92.955023) (width 0.3) (layer "B.Cu") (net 23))
 (segment (start 170.384977 92.955023) (end 169.335023 94.004977) (width 0.3) (layer "B.Cu") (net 23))
 (segment (start 153.54 98.05) (end 153.54 98.1) (width 0.3) (layer "F.Cu") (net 21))
 (segment (start 157.64 93.95) (end 153.54 98.05) (width 0.3) (layer "F.Cu") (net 21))
 (segment (start 157.265 91.035) (end 157.64 91.41) (width 0.3) (layer "F.Cu") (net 20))
 (segment (start 152.4725 91.035) (end 157.265 91.035) (width 0.3) (layer "F.Cu") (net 20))
 (segment (start 156.02452 90.48548) (end 157.64 88.87) (width 0.3) (layer "F.Cu") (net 3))
 (segment (start 147.29702 90.48548) (end 156.02452 90.48548) (width 0.3) (layer "F.Cu") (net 3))
 (segment (start 146.7475 91.035) (end 147.29702 90.48548) (width 0.3) (layer "F.Cu") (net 3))
 (segment (start 152.4725 91.685) (end 155.9205 91.685) (width 0.3) (layer "F.Cu") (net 19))
 (segment (start 155.9205 91.685) (end 156.02 91.7845) (width 0.3) (layer "F.Cu") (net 19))
 (via (at 156.02 91.7845) (size 0.8) (drill 0.4) (layers "F.Cu" "B.Cu") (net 19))
 (segment (start 159.69 91.44) (end 159.72 91.41) (width 0.3) (layer "B.Cu") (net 19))
 (segment (start 157.164345 90.26) (end 158.51 90.26) (width 0.3) (layer "B.Cu") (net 19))
 (segment (start 156.02 91.7845) (end 156.02 91.404345) (width 0.3) (layer "B.Cu") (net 19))
 (segment (start 156.02 91.404345) (end 157.164345 90.26) (width 0.3) (layer "B.Cu") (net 19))
 (segment (start 158.51 90.26) (end 159.69 91.44) (width 0.3) (layer "B.Cu") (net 19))
 (segment (start 159.72 91.41) (end 172.88 91.41) (width 0.3) (layer "B.Cu") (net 19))
 (segment (start 171.344847 90.405153) (end 172.88 88.87) (width 0.3) (layer "F.Cu") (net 4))
 (segment (start 171.344847 92.1595) (end 171.344847 90.405153) (width 0.3) (layer "F.Cu") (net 4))
 (segment (start 150.815 91.685) (end 150.83 91.67) (width 0.3) (layer "F.Cu") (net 4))
 (segment (start 146.7475 91.685) (end 150.815 91.685) (width 0.3) (layer "F.Cu") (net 4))
 (via (at 171.344847 92.1595) (size 0.8) (drill 0.4) (layers "F.Cu" "B.Cu") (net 4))
 (via (at 150.83 91.67) (size 0.8) (drill 0.4) (layers "F.Cu" "B.Cu") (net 4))
 (segment (start 169.740519 92.559511) (end 170.14053 92.1595) (width 0.3) (layer "B.Cu") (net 4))
 (segment (start 170.14053 92.1595) (end 171.344847 92.1595) (width 0.3) (layer "B.Cu") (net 4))
 (segment (start 150.83 91.67) (end 150.83 89.762) (width 0.3) (layer "B.Cu") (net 4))
 (segment (start 154.967511 92.559511) (end 169.740519 92.559511) (width 0.3) (layer "B.Cu") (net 4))
 (segment (start 150.83 89.762) (end 151.5 89.092) (width 0.3) (layer "B.Cu") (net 4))
 (segment (start 151.5 89.092) (end 154.967511 92.559511) (width 0.3) (layer "B.Cu") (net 4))
 (segment (start 169.190489 92.800489) (end 172.88 96.49) (width 0.3) (layer "F.Cu") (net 18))
 (segment (start 155.51053 92.335) (end 155.976019 92.800489) (width 0.3) (layer "F.Cu") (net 18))
 (segment (start 155.976019 92.800489) (end 169.190489 92.800489) (width 0.3) (layer "F.Cu") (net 18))
 (segment (start 152.4725 92.335) (end 155.51053 92.335) (width 0.3) (layer "F.Cu") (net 18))
 (segment (start 153.545 92.985) (end 155.545023 94.985023) (width 0.3) (layer "F.Cu") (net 17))
 (segment (start 152.4725 92.985) (end 153.545 92.985) (width 0.3) (layer "F.Cu") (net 17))
 (via (at 155.545023 94.985023) (size 0.8) (drill 0.4) (layers "F.Cu" "B.Cu") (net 17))
 (segment (start 155.659511 95.099511) (end 158.519511 95.099511) (width 0.3) (layer "B.Cu") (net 17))
 (segment (start 155.545023 94.985023) (end 155.659511 95.099511) (width 0.3) (layer "B.Cu") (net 17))
 (segment (start 158.519511 95.099511) (end 162.45 99.03) (width 0.3) (layer "B.Cu") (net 17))
 (segment (start 162.45 99.03) (end 172.88 99.03) (width 0.3) (layer "B.Cu") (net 17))
 (segment (start 146.7475 92.335) (end 148.045 92.335) (width 0.3) (layer "F.Cu") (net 5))
 (segment (start 148.045 92.335) (end 148.59 92.88) (width 0.3) (layer "F.Cu") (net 5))
 (via (at 148.59 92.88) (size 0.8) (drill 0.4) (layers "F.Cu" "B.Cu") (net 5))
 (segment (start 148.59 92.88) (end 152.2 96.49) (width 0.3) (layer "B.Cu") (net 5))
 (segment (start 152.2 96.49) (end 157.64 96.49) (width 0.3) (layer "B.Cu") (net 5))
 (segment (start 148.96 92.51) (end 148.96 89.092) (width 0.3) (layer "B.Cu") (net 5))
 (segment (start 148.59 92.88) (end 148.96 92.51) (width 0.3) (layer "B.Cu") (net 5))
 (segment (start 148.24 95.82) (end 148.005 95.585) (width 0.3) (layer "F.Cu") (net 9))
 (segment (start 148.24 98.69) (end 148.24 95.82) (width 0.3) (layer "F.Cu") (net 9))
 (segment (start 148.005 95.585) (end 146.7475 95.585) (width 0.3) (layer "F.Cu") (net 9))
 (segment (start 144.91 96.375) (end 145.05 96.235) (width 0.3) (layer "F.Cu") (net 1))
 (segment (start 144.24 97.045) (end 144.91 96.375) (width 0.5) (layer "F.Cu") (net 1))
 (segment (start 132.525 97.69) (end 142.185 97.69) (width 0.5) (layer "F.Cu") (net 1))
 (segment (start 142.185 97.69) (end 142.83 97.045) (width 0.5) (layer "F.Cu") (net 1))
 (segment (start 142.83 97.045) (end 144.24 97.045) (width 0.5) (layer "F.Cu") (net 1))
 (segment (start 145.05 96.235) (end 146.7475 96.235) (width 0.3) (layer "F.Cu") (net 1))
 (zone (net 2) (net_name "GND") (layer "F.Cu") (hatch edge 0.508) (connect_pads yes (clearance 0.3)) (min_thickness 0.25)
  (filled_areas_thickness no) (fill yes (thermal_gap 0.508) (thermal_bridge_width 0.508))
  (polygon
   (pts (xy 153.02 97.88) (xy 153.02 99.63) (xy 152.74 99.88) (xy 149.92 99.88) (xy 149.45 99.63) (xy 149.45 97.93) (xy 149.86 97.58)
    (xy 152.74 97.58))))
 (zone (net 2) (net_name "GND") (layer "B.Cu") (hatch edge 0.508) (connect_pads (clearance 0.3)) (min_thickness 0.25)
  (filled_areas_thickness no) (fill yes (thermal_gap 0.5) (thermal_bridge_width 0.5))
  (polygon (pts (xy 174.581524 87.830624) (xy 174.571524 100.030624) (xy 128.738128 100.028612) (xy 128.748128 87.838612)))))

